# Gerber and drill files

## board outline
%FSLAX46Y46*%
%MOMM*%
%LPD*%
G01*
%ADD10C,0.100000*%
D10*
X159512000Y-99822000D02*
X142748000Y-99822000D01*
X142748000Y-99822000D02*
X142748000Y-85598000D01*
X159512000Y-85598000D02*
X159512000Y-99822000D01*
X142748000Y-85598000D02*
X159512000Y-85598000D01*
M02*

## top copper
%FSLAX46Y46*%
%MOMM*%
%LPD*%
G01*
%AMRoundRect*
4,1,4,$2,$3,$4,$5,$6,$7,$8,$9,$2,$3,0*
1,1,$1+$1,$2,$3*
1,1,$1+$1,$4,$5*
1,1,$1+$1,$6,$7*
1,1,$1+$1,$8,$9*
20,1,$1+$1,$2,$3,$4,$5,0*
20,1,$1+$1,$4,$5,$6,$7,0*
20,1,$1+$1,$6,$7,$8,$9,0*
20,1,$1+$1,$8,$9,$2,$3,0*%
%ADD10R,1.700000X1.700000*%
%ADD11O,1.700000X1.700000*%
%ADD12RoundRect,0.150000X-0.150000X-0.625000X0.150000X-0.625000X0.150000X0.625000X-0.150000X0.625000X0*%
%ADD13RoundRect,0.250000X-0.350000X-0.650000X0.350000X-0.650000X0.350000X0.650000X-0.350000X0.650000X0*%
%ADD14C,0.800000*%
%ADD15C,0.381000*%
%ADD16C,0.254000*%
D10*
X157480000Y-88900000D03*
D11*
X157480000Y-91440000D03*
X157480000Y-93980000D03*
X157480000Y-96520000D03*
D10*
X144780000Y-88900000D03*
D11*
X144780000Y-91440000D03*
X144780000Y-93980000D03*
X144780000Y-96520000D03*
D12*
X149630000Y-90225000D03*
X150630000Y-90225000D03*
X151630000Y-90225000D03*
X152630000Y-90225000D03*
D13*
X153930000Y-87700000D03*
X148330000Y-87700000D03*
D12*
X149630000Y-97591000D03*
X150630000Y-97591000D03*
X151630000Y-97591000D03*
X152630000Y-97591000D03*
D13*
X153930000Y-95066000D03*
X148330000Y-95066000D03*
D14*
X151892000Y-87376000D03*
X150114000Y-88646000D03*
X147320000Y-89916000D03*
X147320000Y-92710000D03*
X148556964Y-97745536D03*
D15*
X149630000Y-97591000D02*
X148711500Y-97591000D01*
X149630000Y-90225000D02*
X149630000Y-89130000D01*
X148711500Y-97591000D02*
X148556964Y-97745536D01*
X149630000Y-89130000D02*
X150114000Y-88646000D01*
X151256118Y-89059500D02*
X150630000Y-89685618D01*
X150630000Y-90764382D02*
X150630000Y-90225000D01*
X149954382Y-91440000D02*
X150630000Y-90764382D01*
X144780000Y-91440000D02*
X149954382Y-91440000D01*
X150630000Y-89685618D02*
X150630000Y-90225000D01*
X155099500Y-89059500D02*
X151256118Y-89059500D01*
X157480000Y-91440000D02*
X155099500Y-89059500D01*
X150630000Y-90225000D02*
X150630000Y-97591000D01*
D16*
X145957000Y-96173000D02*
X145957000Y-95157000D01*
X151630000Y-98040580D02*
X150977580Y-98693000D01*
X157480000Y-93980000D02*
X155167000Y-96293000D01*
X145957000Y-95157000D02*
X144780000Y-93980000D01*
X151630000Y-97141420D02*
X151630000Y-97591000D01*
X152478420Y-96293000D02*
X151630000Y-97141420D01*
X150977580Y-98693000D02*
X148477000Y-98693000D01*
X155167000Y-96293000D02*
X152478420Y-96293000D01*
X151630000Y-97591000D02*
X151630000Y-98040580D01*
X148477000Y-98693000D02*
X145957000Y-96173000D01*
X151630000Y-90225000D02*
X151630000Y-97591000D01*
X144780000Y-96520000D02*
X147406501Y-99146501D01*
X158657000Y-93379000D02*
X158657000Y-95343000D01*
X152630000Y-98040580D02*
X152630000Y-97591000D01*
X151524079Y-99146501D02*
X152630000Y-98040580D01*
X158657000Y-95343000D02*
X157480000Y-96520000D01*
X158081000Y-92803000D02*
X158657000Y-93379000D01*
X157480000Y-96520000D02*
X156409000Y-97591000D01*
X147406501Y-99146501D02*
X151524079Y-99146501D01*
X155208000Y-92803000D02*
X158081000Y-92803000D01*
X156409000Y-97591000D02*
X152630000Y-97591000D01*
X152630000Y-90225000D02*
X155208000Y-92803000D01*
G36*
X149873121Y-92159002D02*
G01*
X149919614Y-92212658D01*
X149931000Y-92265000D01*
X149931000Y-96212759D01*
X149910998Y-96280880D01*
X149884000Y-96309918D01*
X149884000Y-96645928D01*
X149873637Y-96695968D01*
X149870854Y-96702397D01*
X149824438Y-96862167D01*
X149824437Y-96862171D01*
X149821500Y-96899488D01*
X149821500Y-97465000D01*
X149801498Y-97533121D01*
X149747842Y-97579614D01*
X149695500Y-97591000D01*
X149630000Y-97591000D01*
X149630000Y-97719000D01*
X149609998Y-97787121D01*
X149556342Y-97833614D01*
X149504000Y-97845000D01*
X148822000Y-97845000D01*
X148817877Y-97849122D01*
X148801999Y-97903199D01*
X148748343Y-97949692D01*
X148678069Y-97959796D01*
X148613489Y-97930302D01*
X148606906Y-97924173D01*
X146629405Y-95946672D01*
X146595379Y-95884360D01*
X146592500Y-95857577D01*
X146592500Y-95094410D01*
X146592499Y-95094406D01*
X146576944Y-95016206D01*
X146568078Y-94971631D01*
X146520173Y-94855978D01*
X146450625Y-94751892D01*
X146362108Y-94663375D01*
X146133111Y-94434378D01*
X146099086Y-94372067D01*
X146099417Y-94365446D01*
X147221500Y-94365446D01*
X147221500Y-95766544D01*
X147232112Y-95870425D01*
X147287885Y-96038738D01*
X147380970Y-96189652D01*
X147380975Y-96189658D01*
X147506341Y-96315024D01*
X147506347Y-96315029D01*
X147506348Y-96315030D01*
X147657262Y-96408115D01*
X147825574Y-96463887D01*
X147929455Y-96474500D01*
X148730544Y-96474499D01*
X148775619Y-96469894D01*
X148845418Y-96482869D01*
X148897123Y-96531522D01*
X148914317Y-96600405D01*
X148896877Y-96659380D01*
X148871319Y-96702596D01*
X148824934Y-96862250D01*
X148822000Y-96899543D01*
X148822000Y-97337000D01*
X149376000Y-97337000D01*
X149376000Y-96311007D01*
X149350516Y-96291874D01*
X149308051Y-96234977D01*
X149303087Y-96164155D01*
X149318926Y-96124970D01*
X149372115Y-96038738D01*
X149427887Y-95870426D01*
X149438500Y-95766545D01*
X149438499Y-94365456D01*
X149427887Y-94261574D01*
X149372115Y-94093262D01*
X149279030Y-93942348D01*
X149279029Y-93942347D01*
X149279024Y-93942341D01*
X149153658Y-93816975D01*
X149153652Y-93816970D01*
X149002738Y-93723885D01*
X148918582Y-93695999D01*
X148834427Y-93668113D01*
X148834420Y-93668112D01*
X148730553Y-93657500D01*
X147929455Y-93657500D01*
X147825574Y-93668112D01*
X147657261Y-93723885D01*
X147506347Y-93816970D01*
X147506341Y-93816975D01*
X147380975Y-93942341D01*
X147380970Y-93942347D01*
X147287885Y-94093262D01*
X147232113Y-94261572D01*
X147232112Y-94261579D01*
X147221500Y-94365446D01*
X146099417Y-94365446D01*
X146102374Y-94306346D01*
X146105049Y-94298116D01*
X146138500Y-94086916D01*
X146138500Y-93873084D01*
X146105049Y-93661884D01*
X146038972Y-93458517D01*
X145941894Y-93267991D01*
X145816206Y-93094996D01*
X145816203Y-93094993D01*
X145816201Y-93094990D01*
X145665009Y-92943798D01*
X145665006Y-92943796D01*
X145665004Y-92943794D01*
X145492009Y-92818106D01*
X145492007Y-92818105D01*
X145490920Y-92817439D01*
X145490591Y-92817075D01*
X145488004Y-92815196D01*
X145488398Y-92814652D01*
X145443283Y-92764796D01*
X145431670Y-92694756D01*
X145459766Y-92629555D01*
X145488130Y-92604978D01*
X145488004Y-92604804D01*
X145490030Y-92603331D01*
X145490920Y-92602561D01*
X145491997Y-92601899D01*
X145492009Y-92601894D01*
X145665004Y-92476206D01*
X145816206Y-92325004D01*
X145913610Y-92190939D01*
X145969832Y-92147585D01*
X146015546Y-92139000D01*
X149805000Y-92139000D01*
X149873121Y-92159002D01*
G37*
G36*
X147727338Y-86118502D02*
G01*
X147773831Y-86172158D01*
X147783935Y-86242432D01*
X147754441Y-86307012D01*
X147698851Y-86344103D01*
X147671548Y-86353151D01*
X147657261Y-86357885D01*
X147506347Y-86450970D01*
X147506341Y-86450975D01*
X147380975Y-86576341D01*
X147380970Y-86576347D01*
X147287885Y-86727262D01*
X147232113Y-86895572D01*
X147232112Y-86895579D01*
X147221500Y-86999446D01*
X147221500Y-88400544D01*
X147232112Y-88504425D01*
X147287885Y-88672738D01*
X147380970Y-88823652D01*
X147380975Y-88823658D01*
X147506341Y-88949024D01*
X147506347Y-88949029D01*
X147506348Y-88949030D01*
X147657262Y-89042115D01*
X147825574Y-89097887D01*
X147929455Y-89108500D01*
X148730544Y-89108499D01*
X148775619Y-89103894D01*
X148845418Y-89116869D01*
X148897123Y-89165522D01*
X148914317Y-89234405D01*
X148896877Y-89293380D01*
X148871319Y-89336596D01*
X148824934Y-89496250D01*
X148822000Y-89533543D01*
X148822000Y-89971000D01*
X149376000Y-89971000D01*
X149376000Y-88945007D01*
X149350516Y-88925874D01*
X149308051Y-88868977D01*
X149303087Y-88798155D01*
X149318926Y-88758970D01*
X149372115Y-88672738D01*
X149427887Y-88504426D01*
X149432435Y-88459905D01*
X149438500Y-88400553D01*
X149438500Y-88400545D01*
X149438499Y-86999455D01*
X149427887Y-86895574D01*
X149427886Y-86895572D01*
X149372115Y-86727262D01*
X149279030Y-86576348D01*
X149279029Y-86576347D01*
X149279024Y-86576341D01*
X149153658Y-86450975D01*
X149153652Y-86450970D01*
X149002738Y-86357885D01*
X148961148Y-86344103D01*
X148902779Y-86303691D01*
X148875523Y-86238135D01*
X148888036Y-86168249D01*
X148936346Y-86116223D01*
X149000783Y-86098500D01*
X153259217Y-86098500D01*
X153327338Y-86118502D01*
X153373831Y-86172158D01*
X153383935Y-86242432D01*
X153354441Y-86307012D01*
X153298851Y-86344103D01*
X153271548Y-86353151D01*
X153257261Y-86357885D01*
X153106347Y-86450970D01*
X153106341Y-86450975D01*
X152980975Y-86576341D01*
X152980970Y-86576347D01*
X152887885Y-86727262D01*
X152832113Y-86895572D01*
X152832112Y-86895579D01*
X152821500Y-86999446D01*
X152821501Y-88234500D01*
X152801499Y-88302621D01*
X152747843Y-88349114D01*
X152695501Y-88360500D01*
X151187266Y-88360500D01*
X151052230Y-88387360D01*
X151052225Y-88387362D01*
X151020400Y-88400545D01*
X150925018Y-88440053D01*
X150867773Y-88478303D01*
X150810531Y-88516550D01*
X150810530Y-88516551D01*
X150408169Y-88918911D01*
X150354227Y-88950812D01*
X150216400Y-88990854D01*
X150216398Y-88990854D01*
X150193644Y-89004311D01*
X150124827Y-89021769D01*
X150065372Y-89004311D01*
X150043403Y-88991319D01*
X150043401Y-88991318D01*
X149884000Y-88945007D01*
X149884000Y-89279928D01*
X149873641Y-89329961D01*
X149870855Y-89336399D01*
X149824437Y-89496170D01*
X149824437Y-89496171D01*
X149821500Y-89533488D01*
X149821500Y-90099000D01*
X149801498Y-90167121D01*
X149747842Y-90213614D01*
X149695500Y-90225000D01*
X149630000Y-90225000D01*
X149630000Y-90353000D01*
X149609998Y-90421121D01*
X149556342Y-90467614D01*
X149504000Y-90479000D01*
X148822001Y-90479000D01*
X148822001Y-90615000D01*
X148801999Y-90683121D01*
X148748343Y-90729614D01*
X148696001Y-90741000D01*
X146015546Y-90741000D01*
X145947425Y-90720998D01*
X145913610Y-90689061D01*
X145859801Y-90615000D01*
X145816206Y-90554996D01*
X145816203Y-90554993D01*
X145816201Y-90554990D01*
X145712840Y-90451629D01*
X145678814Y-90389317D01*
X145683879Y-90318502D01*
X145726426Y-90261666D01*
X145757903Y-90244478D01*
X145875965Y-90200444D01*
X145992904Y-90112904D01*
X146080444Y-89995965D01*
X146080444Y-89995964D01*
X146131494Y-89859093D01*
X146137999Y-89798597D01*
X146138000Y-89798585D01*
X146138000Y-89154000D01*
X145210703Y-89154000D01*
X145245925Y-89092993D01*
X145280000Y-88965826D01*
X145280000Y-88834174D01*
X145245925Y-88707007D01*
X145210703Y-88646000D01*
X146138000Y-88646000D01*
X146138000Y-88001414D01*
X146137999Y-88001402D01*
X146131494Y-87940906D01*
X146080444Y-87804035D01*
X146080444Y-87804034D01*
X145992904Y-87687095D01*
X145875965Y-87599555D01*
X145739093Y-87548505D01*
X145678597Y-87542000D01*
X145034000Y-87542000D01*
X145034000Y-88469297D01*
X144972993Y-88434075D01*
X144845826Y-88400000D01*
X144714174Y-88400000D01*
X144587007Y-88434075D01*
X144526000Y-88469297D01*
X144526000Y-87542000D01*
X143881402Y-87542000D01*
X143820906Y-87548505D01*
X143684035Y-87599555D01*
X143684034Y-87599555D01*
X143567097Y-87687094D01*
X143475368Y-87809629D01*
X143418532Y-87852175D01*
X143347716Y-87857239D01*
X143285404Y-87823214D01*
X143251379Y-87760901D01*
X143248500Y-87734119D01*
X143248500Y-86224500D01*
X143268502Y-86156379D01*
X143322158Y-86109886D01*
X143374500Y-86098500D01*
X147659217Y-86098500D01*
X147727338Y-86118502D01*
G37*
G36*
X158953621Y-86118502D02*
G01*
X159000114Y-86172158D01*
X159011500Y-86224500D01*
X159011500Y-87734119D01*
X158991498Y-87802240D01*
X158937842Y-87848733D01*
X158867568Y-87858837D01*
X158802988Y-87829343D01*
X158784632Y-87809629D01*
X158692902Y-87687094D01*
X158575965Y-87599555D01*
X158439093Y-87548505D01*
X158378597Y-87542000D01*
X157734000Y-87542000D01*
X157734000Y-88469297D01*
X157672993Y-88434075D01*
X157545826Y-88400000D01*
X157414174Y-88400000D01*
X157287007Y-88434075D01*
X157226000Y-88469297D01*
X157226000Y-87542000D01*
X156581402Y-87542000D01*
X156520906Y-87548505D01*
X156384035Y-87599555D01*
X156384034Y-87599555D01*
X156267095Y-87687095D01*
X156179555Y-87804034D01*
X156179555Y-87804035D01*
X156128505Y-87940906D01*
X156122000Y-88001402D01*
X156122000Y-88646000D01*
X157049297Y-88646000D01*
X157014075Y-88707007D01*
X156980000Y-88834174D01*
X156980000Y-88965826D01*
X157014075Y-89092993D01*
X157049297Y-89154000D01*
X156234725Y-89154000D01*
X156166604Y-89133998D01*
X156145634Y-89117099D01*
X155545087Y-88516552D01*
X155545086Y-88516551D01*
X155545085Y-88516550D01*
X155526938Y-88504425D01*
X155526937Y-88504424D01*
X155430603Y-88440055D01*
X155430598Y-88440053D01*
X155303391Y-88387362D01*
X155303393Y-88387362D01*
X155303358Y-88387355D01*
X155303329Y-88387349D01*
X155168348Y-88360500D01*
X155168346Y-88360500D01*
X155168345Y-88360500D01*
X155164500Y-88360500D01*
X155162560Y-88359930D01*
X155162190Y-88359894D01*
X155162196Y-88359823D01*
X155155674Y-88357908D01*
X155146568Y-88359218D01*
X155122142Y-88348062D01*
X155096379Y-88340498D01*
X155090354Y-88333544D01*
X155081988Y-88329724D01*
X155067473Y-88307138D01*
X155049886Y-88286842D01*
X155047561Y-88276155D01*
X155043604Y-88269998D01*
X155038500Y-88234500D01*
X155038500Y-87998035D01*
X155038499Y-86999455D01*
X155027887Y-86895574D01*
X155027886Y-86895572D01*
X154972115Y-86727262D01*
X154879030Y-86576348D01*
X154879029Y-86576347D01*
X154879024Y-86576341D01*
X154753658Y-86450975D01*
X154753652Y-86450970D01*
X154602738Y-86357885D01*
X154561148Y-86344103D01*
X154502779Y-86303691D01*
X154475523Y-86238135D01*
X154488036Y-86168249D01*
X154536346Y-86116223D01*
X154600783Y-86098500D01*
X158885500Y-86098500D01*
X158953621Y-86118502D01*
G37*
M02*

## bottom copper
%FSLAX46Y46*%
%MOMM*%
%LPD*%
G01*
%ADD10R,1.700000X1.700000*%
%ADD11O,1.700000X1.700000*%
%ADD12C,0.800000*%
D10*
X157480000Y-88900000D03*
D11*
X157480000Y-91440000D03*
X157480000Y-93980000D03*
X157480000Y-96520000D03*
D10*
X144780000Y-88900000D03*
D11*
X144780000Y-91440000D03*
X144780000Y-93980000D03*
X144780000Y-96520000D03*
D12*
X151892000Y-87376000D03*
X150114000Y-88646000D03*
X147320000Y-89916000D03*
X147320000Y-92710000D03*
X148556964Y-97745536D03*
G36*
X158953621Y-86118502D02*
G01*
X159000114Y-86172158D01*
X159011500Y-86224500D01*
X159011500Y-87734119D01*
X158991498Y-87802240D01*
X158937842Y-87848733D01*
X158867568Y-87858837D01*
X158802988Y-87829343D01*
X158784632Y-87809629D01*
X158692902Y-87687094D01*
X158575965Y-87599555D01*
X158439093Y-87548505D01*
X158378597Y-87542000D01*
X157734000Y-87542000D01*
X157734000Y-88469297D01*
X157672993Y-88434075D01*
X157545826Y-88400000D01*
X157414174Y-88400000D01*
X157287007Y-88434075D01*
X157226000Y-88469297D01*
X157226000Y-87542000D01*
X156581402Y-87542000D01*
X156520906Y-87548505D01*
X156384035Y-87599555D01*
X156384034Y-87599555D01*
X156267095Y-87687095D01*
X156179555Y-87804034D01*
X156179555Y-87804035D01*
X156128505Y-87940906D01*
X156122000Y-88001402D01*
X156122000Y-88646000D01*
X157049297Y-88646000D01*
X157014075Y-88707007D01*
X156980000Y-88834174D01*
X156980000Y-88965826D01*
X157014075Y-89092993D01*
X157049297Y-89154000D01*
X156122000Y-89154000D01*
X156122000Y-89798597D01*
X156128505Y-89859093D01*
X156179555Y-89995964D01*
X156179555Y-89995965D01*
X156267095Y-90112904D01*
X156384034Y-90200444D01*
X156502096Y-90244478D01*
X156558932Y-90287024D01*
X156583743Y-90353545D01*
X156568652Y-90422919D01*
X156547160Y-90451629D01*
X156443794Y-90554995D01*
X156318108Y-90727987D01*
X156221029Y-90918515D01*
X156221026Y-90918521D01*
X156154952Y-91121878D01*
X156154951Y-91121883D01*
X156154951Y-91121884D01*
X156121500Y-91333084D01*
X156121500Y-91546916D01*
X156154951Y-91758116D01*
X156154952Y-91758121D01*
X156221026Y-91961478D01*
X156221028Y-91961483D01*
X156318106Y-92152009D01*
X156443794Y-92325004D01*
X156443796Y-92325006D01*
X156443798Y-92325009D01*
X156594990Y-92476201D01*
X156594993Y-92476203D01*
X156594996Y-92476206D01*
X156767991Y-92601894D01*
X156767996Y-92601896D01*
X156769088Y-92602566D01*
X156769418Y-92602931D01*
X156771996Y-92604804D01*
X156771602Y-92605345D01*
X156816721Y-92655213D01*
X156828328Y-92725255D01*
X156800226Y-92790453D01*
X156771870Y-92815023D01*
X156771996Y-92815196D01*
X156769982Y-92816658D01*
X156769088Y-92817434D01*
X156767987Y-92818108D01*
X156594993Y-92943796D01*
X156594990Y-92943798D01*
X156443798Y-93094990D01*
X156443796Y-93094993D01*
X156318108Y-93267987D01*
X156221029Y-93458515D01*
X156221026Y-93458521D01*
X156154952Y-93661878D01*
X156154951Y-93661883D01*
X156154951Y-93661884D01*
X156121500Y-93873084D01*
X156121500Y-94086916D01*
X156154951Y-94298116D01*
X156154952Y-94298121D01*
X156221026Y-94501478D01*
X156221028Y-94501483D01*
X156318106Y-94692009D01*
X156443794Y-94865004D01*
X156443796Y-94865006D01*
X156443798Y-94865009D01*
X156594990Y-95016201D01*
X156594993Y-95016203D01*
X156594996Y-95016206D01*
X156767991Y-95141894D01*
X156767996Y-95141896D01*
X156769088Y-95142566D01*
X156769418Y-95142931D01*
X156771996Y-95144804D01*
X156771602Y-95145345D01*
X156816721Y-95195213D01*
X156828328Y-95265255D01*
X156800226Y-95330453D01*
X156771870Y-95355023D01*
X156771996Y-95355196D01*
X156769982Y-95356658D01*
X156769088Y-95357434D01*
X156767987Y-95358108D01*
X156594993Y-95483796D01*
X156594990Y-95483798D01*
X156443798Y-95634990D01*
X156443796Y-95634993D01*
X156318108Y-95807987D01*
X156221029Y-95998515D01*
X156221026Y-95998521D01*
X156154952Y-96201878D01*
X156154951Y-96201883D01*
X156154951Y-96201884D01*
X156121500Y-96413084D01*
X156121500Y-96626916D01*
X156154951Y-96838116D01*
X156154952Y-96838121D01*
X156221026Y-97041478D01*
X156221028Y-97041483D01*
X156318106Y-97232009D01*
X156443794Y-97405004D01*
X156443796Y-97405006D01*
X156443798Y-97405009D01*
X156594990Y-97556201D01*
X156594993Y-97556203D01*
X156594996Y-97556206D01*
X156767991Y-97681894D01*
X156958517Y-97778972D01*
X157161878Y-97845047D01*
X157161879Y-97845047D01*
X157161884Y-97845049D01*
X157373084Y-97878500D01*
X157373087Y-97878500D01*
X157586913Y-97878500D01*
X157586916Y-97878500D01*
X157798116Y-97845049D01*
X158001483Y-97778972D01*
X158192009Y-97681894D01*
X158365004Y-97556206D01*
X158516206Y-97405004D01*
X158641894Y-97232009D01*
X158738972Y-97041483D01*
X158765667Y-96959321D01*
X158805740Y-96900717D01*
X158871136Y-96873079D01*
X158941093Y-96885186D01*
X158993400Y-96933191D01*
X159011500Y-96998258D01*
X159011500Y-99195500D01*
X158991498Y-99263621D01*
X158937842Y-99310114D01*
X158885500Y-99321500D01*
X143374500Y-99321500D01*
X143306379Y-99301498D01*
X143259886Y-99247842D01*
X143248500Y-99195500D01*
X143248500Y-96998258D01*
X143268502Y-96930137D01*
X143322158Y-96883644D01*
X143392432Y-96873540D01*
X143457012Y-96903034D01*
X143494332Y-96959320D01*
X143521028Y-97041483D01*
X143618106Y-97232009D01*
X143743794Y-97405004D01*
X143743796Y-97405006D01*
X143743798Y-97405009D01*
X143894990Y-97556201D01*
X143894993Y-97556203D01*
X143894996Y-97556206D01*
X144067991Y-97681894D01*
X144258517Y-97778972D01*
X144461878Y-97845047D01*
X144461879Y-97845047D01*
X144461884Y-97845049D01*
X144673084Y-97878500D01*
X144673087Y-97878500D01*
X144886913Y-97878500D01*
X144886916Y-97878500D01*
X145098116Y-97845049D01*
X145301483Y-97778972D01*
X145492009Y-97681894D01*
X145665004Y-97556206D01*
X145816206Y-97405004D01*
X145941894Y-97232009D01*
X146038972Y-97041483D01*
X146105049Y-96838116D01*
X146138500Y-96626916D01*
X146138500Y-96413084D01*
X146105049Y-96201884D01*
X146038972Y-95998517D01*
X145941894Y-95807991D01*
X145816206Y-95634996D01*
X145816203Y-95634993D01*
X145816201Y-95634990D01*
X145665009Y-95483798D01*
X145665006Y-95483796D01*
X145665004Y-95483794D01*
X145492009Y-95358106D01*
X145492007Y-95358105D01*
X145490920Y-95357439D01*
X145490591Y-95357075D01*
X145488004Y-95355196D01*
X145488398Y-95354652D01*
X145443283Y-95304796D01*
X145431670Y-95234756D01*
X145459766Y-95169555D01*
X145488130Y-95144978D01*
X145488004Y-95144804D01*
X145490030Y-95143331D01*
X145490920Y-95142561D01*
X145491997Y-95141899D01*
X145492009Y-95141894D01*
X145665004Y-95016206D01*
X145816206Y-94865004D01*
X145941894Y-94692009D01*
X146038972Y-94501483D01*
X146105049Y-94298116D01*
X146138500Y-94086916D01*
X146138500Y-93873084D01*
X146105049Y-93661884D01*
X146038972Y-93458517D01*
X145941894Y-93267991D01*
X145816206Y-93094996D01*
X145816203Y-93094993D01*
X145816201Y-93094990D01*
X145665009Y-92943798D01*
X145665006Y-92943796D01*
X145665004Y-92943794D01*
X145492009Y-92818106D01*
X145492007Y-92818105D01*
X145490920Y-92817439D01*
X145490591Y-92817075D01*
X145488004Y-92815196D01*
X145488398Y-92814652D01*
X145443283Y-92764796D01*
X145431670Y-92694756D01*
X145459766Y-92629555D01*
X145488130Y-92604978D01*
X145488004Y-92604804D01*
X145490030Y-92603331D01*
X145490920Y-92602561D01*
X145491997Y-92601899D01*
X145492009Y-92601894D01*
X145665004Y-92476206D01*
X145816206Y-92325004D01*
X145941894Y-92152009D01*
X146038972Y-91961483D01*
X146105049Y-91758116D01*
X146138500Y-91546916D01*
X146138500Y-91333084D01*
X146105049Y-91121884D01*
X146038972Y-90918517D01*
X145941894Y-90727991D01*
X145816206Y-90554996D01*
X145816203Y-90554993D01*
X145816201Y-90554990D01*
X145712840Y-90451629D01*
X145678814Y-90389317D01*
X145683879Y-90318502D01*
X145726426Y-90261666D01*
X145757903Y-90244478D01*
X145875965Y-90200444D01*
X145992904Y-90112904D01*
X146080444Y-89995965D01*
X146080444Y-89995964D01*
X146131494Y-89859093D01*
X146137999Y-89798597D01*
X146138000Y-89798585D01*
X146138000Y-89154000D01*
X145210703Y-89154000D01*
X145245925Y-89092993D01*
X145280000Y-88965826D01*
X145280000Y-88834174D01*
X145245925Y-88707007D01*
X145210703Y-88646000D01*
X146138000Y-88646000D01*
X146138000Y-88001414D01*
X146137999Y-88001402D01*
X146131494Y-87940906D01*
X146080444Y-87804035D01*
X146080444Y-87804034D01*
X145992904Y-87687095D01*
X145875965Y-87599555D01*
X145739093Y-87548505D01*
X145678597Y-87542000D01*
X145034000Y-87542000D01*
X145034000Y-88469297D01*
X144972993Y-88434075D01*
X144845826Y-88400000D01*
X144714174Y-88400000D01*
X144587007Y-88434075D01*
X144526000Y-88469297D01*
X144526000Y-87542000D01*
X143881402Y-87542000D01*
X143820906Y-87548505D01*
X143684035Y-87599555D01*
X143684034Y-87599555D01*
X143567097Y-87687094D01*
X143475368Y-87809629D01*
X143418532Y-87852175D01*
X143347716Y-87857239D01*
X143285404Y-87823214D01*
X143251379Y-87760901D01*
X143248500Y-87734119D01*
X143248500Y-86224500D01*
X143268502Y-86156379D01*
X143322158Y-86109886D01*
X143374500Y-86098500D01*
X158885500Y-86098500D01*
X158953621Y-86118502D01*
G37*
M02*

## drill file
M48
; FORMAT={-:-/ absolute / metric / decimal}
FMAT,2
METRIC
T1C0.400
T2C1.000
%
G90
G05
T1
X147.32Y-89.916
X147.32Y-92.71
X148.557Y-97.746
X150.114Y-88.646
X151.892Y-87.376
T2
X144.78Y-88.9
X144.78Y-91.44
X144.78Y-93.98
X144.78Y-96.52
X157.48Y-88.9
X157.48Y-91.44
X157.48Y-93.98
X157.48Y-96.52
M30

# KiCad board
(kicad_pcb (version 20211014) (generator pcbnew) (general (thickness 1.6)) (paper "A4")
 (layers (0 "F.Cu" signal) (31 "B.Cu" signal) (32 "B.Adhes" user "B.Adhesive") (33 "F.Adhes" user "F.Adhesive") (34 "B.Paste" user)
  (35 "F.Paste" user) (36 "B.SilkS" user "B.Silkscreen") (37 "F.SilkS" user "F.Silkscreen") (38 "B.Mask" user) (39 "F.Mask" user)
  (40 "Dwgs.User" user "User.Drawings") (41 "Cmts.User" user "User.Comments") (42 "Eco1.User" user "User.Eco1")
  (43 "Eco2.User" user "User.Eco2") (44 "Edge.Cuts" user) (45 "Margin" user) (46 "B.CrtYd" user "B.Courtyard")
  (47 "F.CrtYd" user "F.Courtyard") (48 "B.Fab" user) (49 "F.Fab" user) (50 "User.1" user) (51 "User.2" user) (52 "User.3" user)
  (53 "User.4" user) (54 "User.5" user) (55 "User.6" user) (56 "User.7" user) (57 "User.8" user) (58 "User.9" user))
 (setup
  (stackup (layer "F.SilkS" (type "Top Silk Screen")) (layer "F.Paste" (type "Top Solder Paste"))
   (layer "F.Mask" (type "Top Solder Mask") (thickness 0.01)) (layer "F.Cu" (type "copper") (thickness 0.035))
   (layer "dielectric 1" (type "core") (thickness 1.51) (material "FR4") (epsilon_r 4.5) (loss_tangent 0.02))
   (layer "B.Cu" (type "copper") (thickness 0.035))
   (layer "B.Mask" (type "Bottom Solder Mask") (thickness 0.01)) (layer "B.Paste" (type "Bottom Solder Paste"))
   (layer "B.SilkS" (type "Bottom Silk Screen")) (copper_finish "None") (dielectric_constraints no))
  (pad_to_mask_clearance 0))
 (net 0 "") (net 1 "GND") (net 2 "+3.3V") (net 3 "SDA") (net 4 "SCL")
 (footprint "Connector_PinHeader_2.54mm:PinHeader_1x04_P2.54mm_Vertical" (layer "F.Cu") (at 157.48 88.9)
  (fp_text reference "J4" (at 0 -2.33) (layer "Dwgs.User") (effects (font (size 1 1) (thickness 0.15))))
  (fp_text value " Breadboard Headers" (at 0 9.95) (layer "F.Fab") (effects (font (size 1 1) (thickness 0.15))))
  (pad "1" thru_hole rect (at 0 0) (size 1.7 1.7) (drill 1) (layers *.Cu *.Mask) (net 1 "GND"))
  (pad "2" thru_hole oval (at 0 2.54) (size 1.7 1.7) (drill 1) (layers *.Cu *.Mask) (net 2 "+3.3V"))
  (pad "3" thru_hole oval (at 0 5.08) (size 1.7 1.7) (drill 1) (layers *.Cu *.Mask) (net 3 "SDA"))
  (pad "4" thru_hole oval (at 0 7.62) (size 1.7 1.7) (drill 1) (layers *.Cu *.Mask) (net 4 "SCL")))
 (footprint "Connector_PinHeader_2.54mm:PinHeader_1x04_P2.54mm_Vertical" (layer "F.Cu") (at 144.78 88.9)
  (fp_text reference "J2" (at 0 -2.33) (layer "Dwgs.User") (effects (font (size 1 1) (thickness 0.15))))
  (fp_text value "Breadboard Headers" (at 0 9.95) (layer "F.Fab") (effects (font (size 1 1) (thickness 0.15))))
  (pad "1" thru_hole rect (at 0 0) (size 1.7 1.7) (drill 1) (layers *.Cu *.Mask) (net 1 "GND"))
  (pad "2" thru_hole oval (at 0 2.54) (size 1.7 1.7) (drill 1) (layers *.Cu *.Mask) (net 2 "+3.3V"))
  (pad "3" thru_hole oval (at 0 5.08) (size 1.7 1.7) (drill 1) (layers *.Cu *.Mask) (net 3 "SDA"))
  (pad "4" thru_hole oval (at 0 7.62) (size 1.7 1.7) (drill 1) (layers *.Cu *.Mask) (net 4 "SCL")))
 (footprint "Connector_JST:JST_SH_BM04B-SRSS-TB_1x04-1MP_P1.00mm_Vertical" (layer "F.Cu") (at 151.13 88.9)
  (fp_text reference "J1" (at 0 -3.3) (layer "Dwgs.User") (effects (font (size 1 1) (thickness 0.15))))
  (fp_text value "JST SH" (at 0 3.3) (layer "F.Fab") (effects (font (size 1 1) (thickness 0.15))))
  (pad "1" smd roundrect (at -1.5 1.325) (size 0.6 1.55) (layers "F.Cu" "F.Paste" "F.Mask") (roundrect_rratio 0.25) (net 1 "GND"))
  (pad "2" smd roundrect (at -0.5 1.325) (size 0.6 1.55) (layers "F.Cu" "F.Paste" "F.Mask") (roundrect_rratio 0.25) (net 2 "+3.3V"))
  (pad "3" smd roundrect (at 0.5 1.325) (size 0.6 1.55) (layers "F.Cu" "F.Paste" "F.Mask") (roundrect_rratio 0.25) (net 3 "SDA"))
  (pad "4" smd roundrect (at 1.5 1.325) (size 0.6 1.55) (layers "F.Cu" "F.Paste" "F.Mask") (roundrect_rratio 0.25) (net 4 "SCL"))
  (pad "MP" smd roundrect (at 2.8 -1.2) (size 1.2 1.8) (layers "F.Cu" "F.Paste" "F.Mask") (roundrect_rratio 0.2083333333))
  (pad "MP" smd roundrect (at -2.8 -1.2) (size 1.2 1.8) (layers "F.Cu" "F.Paste" "F.Mask") (roundrect_rratio 0.2083333333)))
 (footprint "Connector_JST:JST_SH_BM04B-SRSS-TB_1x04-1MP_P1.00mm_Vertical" (layer "F.Cu") (at 151.13 96.266)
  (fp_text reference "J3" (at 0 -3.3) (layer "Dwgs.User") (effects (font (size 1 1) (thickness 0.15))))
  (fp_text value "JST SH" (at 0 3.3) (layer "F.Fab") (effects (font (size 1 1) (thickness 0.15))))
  (pad "1" smd roundrect (at -1.5 1.325) (size 0.6 1.55) (layers "F.Cu" "F.Paste" "F.Mask") (roundrect_rratio 0.25) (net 1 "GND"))
  (pad "2" smd roundrect (at -0.5 1.325) (size 0.6 1.55) (layers "F.Cu" "F.Paste" "F.Mask") (roundrect_rratio 0.25) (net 2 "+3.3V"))
  (pad "3" smd roundrect (at 0.5 1.325) (size 0.6 1.55) (layers "F.Cu" "F.Paste" "F.Mask") (roundrect_rratio 0.25) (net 3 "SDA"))
  (pad "4" smd roundrect (at 1.5 1.325) (size 0.6 1.55) (layers "F.Cu" "F.Paste" "F.Mask") (roundrect_rratio 0.25) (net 4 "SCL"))
  (pad "MP" smd roundrect (at 2.8 -1.2) (size 1.2 1.8) (layers "F.Cu" "F.Paste" "F.Mask") (roundrect_rratio 0.2083333333))
  (pad "MP" smd roundrect (at -2.8 -1.2) (size 1.2 1.8) (layers "F.Cu" "F.Paste" "F.Mask") (roundrect_rratio 0.2083333333)))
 (gr_line (start 159.512 99.822) (end 142.748 99.822) (layer "Edge.Cuts") (width 0.1))
 (gr_line (start 142.748 99.822) (end 142.748 85.598) (layer "Edge.Cuts") (width 0.1))
 (gr_line (start 159.512 85.598) (end 159.512 99.822) (layer "Edge.Cuts") (width 0.1))
 (gr_line (start 142.748 85.598) (end 159.512 85.598) (layer "Edge.Cuts") (width 0.1))
 (segment (start 149.63 97.591) (end 148.7115 97.591) (width 0.381) (layer "F.Cu") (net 1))
 (segment (start 149.63 90.225) (end 149.63 89.13) (width 0.381) (layer "F.Cu") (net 1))
 (segment (start 148.7115 97.591) (end 148.556964 97.745536) (width 0.381) (layer "F.Cu") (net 1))
 (segment (start 149.63 89.13) (end 150.114 88.646) (width 0.381) (layer "F.Cu") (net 1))
 (via (at 151.892 87.376) (size 0.8) (drill 0.4) (layers "F.Cu" "B.Cu") (free) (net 1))
 (via (at 150.114 88.646) (size 0.8) (drill 0.4) (layers "F.Cu" "B.Cu") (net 1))
 (via (at 147.32 89.916) (size 0.8) (drill 0.4) (layers "F.Cu" "B.Cu") (free) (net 1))
 (via (at 147.32 92.71) (size 0.8) (drill 0.4) (layers "F.Cu" "B.Cu") (free) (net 1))
 (via (at 148.556964 97.745536) (size 0.8) (drill 0.4) (layers "F.Cu" "B.Cu") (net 1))
 (segment (start 151.256118 89.0595) (end 150.63 89.685618) (width 0.381) (layer "F.Cu") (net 2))
 (segment (start 150.63 90.764382) (end 150.63 90.225) (width 0.381) (layer "F.Cu") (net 2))
 (segment (start 149.954382 91.44) (end 150.63 90.764382) (width 0.381) (layer "F.Cu") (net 2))
 (segment (start 144.78 91.44) (end 149.954382 91.44) (width 0.381) (layer "F.Cu") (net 2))
 (segment (start 150.63 89.685618) (end 150.63 90.225) (width 0.381) (layer "F.Cu") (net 2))
 (segment (start 155.0995 89.0595) (end 151.256118 89.0595) (width 0.381) (layer "F.Cu") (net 2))
 (segment (start 157.48 91.44) (end 155.0995 89.0595) (width 0.381) (layer "F.Cu") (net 2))
 (segment (start 150.63 90.225) (end 150.63 97.591) (width 0.381) (layer "F.Cu") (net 2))
 (segment (start 145.957 96.173) (end 145.957 95.157) (width 0.254) (layer "F.Cu") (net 3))
 (segment (start 151.63 98.04058) (end 150.97758 98.693) (width 0.254) (layer "F.Cu") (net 3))
 (segment (start 157.48 93.98) (end 155.167 96.293) (width 0.254) (layer "F.Cu") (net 3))
 (segment (start 145.957 95.157) (end 144.78 93.98) (width 0.254) (layer "F.Cu") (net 3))
 (segment (start 151.63 97.14142) (end 151.63 97.591) (width 0.254) (layer "F.Cu") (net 3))
 (segment (start 152.47842 96.293) (end 151.63 97.14142) (width 0.254) (layer "F.Cu") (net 3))
 (segment (start 150.97758 98.693) (end 148.477 98.693) (width 0.254) (layer "F.Cu") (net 3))
 (segment (start 155.167 96.293) (end 152.47842 96.293) (width 0.254) (layer "F.Cu") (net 3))
 (segment (start 151.63 97.591) (end 151.63 98.04058) (width 0.254) (layer "F.Cu") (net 3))
 (segment (start 148.477 98.693) (end 145.957 96.173) (width 0.254) (layer "F.Cu") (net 3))
 (segment (start 151.63 90.225) (end 151.63 97.591) (width 0.254) (layer "F.Cu") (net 3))
 (segment (start 144.78 96.52) (end 147.406501 99.146501) (width 0.254) (layer "F.Cu") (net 4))
 (segment (start 158.657 93.379) (end 158.657 95.343) (width 0.254) (layer "F.Cu") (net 4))
 (segment (start 152.63 98.04058) (end 152.63 97.591) (width 0.254) (layer "F.Cu") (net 4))
 (segment (start 151.524079 99.146501) (end 152.63 98.04058) (width 0.254) (layer "F.Cu") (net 4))
 (segment (start 158.657 95.343) (end 157.48 96.52) (width 0.254) (layer "F.Cu") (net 4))
 (segment (start 158.081 92.803) (end 158.657 93.379) (width 0.254) (layer "F.Cu") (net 4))
 (segment (start 157.48 96.52) (end 156.409 97.591) (width 0.254) (layer "F.Cu") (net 4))
 (segment (start 147.406501 99.146501) (end 151.524079 99.146501) (width 0.254) (layer "F.Cu") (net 4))
 (segment (start 155.208 92.803) (end 158.081 92.803) (width 0.254) (layer "F.Cu") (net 4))
 (segment (start 156.409 97.591) (end 152.63 97.591) (width 0.254) (layer "F.Cu") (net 4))
 (segment (start 152.63 90.225) (end 155.208 92.803) (width 0.254) (layer "F.Cu") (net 4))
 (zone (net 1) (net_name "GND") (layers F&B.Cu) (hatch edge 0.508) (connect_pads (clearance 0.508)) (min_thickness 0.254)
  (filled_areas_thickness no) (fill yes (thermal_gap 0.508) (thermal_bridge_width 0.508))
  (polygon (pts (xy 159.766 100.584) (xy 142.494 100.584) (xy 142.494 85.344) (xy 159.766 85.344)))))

